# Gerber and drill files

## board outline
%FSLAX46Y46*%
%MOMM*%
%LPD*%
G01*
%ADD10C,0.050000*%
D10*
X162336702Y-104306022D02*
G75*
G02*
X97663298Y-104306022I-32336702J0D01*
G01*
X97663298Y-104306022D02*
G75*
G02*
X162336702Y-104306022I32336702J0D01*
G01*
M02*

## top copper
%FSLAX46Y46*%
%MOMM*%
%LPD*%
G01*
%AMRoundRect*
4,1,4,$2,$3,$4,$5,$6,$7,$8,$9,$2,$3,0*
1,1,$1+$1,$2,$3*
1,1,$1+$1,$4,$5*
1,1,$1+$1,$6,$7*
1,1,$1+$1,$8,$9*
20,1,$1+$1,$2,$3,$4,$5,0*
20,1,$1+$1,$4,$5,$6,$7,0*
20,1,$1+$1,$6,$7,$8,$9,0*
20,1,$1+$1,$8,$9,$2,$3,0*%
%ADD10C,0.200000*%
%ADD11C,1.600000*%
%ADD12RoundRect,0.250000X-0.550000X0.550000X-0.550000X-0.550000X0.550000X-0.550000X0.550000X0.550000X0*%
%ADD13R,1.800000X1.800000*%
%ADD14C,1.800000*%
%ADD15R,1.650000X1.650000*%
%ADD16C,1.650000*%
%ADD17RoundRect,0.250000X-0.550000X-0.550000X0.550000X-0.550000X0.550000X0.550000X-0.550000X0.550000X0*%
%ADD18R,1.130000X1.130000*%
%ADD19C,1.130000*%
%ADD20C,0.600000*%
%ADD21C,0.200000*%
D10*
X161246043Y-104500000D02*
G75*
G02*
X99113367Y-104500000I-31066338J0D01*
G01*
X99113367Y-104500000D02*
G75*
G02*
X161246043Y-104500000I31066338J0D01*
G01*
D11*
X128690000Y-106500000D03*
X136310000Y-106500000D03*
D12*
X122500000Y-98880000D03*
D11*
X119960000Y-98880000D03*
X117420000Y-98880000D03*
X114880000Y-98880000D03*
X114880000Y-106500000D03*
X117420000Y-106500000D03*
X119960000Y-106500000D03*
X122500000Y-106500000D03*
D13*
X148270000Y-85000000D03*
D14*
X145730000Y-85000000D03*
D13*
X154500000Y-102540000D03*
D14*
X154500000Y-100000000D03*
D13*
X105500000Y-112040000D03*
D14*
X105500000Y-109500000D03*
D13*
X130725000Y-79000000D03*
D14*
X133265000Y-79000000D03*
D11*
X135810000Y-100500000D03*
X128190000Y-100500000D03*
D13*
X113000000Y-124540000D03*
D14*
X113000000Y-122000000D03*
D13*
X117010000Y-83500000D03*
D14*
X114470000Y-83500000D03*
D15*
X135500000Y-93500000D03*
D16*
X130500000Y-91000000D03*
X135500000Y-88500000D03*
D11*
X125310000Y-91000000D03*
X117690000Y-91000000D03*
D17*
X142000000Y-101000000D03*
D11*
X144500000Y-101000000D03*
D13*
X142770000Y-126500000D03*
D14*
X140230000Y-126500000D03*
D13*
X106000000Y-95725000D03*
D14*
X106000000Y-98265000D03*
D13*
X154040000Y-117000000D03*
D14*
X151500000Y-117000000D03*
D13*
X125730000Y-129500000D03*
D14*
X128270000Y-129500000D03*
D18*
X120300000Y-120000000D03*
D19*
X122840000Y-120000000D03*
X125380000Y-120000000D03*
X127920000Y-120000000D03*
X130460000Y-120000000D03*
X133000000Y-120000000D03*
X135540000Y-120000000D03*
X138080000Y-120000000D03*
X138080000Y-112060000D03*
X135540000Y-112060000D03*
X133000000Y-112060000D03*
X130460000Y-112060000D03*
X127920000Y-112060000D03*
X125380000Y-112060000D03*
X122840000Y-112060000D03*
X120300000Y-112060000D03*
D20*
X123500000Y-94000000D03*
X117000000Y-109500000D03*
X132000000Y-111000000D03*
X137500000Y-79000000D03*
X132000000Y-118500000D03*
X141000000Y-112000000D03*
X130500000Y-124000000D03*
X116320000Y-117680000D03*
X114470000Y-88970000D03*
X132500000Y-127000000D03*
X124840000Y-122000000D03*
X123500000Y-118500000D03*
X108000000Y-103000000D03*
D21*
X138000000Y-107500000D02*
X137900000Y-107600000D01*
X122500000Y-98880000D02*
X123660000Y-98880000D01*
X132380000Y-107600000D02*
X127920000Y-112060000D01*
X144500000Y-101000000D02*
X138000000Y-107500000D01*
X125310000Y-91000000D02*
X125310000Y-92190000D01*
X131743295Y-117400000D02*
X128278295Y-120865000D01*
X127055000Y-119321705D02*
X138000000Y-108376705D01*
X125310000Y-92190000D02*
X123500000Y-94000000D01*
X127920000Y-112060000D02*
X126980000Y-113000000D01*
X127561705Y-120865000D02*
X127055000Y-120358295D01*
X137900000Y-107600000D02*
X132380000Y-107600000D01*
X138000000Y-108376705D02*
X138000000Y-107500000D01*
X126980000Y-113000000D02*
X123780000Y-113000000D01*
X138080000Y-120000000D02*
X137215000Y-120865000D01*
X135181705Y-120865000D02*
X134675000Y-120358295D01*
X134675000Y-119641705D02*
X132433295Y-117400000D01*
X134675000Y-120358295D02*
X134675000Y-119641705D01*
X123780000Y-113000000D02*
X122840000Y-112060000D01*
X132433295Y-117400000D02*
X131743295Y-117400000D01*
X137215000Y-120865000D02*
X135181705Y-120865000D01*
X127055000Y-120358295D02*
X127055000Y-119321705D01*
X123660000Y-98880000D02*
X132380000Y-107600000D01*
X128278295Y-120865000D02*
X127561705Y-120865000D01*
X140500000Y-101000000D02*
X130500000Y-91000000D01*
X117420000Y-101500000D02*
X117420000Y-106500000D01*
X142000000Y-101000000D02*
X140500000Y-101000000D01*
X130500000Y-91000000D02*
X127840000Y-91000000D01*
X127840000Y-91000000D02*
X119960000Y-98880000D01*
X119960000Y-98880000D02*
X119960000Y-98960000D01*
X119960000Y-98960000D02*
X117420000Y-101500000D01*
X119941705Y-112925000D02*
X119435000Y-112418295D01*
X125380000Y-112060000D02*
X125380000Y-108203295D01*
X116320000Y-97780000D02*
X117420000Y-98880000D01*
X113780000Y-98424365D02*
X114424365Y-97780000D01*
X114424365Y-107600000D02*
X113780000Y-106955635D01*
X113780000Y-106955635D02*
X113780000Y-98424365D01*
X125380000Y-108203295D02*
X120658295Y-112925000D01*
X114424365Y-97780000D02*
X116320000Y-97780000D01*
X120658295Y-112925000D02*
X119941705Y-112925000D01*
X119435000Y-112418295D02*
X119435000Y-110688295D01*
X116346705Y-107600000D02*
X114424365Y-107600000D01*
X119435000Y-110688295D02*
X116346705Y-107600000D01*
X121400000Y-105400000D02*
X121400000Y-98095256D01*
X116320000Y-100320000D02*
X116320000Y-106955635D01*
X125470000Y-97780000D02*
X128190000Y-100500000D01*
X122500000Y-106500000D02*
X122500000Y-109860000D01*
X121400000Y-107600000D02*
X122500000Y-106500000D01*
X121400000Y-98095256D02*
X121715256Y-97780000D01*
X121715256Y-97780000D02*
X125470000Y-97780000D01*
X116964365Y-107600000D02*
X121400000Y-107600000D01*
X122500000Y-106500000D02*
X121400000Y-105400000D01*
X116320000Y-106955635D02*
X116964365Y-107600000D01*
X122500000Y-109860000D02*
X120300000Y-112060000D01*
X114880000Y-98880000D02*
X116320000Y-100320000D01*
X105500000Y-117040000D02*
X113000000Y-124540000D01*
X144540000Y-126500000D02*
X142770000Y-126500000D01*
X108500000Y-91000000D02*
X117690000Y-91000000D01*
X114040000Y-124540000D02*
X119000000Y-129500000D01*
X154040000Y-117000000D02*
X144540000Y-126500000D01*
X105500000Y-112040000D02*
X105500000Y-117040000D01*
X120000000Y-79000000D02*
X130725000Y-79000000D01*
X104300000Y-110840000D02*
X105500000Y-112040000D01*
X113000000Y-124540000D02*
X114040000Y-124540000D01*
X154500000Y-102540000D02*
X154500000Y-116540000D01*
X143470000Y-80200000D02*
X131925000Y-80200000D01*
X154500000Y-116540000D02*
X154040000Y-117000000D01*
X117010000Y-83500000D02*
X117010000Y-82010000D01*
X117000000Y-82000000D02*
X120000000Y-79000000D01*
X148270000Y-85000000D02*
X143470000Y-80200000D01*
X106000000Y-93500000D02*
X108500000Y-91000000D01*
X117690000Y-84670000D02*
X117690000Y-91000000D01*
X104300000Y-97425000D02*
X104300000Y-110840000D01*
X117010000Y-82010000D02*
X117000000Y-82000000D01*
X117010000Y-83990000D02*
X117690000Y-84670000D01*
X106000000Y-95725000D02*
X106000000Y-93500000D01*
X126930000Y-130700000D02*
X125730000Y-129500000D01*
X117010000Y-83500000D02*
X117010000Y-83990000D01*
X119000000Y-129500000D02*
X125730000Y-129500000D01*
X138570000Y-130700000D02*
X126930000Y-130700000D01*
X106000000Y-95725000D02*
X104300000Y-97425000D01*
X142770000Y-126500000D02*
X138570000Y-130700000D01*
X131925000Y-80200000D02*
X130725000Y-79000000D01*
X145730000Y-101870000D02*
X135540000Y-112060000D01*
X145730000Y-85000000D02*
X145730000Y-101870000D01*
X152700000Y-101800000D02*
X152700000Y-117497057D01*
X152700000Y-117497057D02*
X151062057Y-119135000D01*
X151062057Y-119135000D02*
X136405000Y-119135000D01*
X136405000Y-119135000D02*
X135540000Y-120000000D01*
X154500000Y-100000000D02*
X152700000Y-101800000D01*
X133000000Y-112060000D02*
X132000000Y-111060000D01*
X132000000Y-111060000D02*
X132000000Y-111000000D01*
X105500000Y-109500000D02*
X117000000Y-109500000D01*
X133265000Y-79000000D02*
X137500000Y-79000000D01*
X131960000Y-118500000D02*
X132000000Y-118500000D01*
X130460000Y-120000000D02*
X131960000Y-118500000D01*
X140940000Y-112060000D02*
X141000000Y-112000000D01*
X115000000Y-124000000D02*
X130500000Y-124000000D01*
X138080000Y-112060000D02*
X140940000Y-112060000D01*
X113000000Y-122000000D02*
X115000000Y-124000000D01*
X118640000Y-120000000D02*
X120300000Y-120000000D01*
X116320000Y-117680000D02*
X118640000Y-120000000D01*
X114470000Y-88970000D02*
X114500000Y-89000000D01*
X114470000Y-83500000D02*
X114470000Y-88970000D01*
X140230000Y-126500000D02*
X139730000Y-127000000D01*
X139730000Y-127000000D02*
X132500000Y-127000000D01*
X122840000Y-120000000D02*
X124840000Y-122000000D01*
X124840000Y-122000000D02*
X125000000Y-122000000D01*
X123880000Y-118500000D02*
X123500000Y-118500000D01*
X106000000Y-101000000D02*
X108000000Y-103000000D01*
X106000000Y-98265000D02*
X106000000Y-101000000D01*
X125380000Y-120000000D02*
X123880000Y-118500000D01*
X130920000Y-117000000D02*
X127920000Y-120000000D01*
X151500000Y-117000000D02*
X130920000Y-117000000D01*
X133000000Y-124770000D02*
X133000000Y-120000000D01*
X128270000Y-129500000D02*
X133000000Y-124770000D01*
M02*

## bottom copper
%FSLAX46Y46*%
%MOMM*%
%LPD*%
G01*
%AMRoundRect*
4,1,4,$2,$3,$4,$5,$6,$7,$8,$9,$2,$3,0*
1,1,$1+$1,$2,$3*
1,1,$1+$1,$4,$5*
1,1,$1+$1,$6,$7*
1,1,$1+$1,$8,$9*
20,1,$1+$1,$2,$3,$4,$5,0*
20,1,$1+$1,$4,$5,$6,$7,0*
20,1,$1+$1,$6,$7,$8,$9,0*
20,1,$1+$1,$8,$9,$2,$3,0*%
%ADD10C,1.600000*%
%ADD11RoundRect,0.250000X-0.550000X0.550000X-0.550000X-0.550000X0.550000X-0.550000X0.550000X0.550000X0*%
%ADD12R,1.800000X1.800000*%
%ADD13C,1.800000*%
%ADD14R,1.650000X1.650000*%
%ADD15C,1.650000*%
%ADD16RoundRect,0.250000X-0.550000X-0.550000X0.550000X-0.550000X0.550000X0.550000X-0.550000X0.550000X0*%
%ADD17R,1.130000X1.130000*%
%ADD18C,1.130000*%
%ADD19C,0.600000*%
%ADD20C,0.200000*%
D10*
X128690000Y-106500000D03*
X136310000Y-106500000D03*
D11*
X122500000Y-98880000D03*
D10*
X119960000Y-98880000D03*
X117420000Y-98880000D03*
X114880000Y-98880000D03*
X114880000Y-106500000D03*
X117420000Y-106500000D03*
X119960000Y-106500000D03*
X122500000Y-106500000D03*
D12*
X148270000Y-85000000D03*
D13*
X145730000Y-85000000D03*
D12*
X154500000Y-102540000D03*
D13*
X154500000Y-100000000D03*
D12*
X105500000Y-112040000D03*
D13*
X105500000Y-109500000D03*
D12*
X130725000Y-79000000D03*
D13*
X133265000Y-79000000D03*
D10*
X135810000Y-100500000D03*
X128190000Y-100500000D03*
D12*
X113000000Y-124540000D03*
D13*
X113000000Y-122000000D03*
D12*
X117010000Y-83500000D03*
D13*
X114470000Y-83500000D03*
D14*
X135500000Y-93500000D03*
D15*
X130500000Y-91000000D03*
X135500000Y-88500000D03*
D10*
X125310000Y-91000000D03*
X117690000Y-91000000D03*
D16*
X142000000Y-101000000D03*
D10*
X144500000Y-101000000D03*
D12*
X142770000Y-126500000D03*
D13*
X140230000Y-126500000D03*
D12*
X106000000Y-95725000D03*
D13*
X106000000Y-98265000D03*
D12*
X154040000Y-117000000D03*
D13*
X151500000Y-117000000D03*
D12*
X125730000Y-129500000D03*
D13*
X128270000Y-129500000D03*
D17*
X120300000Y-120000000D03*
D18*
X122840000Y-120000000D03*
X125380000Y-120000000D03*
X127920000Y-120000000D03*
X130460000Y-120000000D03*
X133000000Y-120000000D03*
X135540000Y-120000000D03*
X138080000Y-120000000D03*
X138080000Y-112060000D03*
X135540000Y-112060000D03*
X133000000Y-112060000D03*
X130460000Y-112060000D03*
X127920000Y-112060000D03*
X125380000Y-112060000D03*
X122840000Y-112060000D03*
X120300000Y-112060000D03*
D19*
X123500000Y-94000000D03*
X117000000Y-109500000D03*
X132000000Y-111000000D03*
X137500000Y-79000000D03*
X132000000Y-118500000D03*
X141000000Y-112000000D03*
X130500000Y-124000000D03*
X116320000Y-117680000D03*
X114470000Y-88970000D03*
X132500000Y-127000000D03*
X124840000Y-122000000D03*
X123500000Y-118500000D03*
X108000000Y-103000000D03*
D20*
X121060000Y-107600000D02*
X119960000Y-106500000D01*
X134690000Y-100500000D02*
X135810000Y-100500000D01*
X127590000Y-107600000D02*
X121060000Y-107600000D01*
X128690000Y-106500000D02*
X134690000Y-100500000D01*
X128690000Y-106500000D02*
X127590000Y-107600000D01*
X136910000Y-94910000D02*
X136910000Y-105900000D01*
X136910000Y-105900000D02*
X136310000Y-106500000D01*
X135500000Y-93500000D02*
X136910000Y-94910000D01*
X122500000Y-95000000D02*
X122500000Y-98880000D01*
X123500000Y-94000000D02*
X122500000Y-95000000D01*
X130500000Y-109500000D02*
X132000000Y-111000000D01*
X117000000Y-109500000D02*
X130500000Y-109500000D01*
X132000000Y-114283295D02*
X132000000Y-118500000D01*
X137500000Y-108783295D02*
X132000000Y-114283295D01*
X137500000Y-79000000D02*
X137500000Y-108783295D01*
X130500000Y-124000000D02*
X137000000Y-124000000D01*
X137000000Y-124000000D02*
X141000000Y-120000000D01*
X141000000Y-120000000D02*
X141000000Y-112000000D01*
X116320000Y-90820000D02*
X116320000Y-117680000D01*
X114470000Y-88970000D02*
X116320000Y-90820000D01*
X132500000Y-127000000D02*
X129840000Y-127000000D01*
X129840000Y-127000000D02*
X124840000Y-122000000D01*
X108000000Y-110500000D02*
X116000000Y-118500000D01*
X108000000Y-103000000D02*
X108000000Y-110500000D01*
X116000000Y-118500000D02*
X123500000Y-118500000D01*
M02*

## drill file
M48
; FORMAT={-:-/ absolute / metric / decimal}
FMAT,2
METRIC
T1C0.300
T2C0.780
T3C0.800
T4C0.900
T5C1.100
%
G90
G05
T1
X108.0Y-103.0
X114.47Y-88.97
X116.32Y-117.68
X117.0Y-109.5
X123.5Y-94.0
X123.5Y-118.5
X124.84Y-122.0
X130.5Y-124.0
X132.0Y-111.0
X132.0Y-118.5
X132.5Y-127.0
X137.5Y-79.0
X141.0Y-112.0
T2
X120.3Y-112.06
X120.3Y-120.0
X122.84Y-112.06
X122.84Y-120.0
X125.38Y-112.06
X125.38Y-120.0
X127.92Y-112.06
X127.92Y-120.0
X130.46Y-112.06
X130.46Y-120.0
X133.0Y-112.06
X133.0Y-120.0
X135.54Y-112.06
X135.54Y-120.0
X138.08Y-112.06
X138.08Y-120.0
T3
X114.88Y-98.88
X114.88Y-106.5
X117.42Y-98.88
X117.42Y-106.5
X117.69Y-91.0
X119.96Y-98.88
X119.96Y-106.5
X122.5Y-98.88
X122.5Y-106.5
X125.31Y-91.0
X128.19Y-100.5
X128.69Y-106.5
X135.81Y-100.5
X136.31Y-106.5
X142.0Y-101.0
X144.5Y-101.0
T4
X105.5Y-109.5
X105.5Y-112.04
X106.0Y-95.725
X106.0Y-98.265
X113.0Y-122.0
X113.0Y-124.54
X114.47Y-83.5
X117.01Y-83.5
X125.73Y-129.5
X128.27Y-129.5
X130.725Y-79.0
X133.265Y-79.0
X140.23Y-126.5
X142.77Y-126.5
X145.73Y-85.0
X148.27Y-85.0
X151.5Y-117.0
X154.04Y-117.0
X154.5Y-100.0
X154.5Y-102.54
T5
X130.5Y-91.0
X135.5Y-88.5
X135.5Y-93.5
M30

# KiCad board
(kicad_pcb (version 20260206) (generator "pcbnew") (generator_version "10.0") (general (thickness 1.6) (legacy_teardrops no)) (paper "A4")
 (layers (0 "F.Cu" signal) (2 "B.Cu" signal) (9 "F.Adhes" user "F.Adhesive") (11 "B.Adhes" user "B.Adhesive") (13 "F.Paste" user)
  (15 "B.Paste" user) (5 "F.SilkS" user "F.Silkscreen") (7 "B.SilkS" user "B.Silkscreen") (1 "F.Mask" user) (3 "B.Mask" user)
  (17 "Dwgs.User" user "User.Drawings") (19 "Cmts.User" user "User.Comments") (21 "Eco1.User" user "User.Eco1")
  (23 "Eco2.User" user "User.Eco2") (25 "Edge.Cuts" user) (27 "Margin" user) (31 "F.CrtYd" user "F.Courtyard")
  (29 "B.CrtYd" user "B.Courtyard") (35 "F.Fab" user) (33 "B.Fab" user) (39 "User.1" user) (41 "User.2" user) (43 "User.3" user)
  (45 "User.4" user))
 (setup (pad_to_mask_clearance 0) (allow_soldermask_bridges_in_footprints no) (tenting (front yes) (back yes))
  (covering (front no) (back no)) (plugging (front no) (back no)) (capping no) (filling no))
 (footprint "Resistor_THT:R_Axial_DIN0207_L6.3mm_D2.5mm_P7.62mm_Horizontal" (layer "F.Cu") (at 128.69 106.5)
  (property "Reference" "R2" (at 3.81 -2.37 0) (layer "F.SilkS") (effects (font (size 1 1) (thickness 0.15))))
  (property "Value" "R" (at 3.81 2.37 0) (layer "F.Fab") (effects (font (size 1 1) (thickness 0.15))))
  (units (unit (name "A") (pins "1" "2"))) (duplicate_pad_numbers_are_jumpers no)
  (pad "1" thru_hole circle (at 0 0) (size 1.6 1.6) (drill 0.8) (layers "*.Cu" "*.Mask") (remove_unused_layers no) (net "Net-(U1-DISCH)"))
  (pad "2" thru_hole circle (at 7.62 0) (size 1.6 1.6) (drill 0.8) (layers "*.Cu" "*.Mask") (remove_unused_layers no) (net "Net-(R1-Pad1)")))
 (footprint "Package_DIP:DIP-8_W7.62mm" (layer "F.Cu") (at 122.5 98.88 -90)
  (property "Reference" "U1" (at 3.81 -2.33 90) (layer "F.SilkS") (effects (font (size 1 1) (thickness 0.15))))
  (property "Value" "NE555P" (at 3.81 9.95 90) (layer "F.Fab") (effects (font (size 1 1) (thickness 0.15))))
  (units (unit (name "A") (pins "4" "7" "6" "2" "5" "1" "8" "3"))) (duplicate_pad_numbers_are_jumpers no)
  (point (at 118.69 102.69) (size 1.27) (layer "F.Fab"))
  (pad "1" thru_hole roundrect (at 0 0 270) (size 1.6 1.6) (drill 0.8) (layers "*.Cu" "*.Mask") (remove_unused_layers no)
   (roundrect_rratio 0.15625) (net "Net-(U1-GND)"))
  (pad "2" thru_hole circle (at 0 2.54 270) (size 1.6 1.6) (drill 0.8) (layers "*.Cu" "*.Mask") (remove_unused_layers no)
   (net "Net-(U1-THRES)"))
  (pad "3" thru_hole circle (at 0 5.08 270) (size 1.6 1.6) (drill 0.8) (layers "*.Cu" "*.Mask") (remove_unused_layers no)
   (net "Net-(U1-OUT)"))
  (pad "4" thru_hole circle (at 0 7.62 270) (size 1.6 1.6) (drill 0.8) (layers "*.Cu" "*.Mask") (remove_unused_layers no)
   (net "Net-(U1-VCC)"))
  (pad "5" thru_hole circle (at 7.62 7.62 270) (size 1.6 1.6) (drill 0.8) (layers "*.Cu" "*.Mask") (remove_unused_layers no)
   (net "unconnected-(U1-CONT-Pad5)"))
  (pad "6" thru_hole circle (at 7.62 5.08 270) (size 1.6 1.6) (drill 0.8) (layers "*.Cu" "*.Mask") (remove_unused_layers no)
   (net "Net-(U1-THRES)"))
  (pad "7" thru_hole circle (at 7.62 2.54 270) (size 1.6 1.6) (drill 0.8) (layers "*.Cu" "*.Mask") (remove_unused_layers no)
   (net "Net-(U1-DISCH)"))
  (pad "8" thru_hole circle (at 7.62 0 270) (size 1.6 1.6) (drill 0.8) (layers "*.Cu" "*.Mask") (remove_unused_layers no)
   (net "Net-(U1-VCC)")))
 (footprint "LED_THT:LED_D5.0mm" (layer "F.Cu") (at 148.27 85 180)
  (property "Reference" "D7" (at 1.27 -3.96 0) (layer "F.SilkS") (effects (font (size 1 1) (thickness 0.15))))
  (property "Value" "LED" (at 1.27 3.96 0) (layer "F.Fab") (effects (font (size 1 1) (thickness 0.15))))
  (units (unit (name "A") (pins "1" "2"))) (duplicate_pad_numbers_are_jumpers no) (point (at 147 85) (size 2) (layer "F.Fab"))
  (pad "1" thru_hole rect (at 0 0 180) (size 1.8 1.8) (drill 0.9) (layers "*.Cu" "*.Mask") (remove_unused_layers no) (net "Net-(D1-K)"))
  (pad "2" thru_hole circle (at 2.54 0 180) (size 1.8 1.8) (drill 0.9) (layers "*.Cu" "*.Mask") (remove_unused_layers no) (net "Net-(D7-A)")))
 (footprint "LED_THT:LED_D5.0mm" (layer "F.Cu") (at 154.5 102.54 90)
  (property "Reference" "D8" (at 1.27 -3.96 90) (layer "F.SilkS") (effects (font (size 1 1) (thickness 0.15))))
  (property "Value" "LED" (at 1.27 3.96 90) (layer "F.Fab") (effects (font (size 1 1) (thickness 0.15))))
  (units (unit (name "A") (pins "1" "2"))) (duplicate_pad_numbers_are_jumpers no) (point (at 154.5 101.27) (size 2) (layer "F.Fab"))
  (pad "1" thru_hole rect (at 0 0 90) (size 1.8 1.8) (drill 0.9) (layers "*.Cu" "*.Mask") (remove_unused_layers no) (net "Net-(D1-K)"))
  (pad "2" thru_hole circle (at 2.54 0 90) (size 1.8 1.8) (drill 0.9) (layers "*.Cu" "*.Mask") (remove_unused_layers no) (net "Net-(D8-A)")))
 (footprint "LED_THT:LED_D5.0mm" (layer "F.Cu") (at 105.5 112.04 90)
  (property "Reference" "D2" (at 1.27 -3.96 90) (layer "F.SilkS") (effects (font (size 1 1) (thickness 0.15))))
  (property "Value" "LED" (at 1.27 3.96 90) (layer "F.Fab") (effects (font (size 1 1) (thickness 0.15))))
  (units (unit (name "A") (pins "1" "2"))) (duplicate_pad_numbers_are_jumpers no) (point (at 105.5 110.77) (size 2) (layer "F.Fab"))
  (pad "1" thru_hole rect (at 0 0 90) (size 1.8 1.8) (drill 0.9) (layers "*.Cu" "*.Mask") (remove_unused_layers no) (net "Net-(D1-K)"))
  (pad "2" thru_hole circle (at 2.54 0 90) (size 1.8 1.8) (drill 0.9) (layers "*.Cu" "*.Mask") (remove_unused_layers no) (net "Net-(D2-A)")))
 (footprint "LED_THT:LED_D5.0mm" (layer "F.Cu") (at 130.725 79)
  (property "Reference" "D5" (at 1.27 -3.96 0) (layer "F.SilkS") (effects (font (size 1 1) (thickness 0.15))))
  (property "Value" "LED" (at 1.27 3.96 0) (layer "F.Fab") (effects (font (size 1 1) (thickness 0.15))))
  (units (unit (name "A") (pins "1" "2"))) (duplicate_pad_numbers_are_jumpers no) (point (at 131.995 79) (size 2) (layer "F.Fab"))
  (pad "1" thru_hole rect (at 0 0) (size 1.8 1.8) (drill 0.9) (layers "*.Cu" "*.Mask") (remove_unused_layers no) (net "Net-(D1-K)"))
  (pad "2" thru_hole circle (at 2.54 0) (size 1.8 1.8) (drill 0.9) (layers "*.Cu" "*.Mask") (remove_unused_layers no) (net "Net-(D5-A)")))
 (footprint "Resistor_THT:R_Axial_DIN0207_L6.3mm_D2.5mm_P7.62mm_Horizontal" (layer "F.Cu") (at 135.81 100.5 180)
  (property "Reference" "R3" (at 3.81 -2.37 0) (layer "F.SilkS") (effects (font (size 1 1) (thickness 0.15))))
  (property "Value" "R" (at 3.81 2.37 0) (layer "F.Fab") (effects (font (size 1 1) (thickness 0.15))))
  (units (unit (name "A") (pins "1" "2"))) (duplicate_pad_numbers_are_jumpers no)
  (pad "1" thru_hole circle (at 0 0 180) (size 1.6 1.6) (drill 0.8) (layers "*.Cu" "*.Mask") (remove_unused_layers no)
   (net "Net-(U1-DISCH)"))
  (pad "2" thru_hole circle (at 7.62 0 180) (size 1.6 1.6) (drill 0.8) (layers "*.Cu" "*.Mask") (remove_unused_layers no)
   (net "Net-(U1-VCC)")))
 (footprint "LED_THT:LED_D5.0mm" (layer "F.Cu") (at 113 124.54 90)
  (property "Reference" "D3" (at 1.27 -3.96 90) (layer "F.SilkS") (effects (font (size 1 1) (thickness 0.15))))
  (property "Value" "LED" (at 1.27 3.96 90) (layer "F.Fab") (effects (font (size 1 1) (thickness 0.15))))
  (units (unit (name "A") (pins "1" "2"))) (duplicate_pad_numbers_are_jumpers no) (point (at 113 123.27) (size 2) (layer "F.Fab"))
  (pad "1" thru_hole rect (at 0 0 90) (size 1.8 1.8) (drill 0.9) (layers "*.Cu" "*.Mask") (remove_unused_layers no) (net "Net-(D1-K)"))
  (pad "2" thru_hole circle (at 2.54 0 90) (size 1.8 1.8) (drill 0.9) (layers "*.Cu" "*.Mask") (remove_unused_layers no) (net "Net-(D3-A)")))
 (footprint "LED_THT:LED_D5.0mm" (layer "F.Cu") (at 117.01 83.5 180)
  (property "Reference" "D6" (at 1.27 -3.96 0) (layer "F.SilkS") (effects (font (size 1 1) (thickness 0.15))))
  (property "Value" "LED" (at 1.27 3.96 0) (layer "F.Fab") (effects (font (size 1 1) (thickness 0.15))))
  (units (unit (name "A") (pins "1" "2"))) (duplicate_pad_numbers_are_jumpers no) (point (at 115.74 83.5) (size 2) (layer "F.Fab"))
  (pad "1" thru_hole rect (at 0 0 180) (size 1.8 1.8) (drill 0.9) (layers "*.Cu" "*.Mask") (remove_unused_layers no) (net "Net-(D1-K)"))
  (pad "2" thru_hole circle (at 2.54 0 180) (size 1.8 1.8) (drill 0.9) (layers "*.Cu" "*.Mask") (remove_unused_layers no) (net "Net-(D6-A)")))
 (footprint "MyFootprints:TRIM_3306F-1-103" (layer "F.Cu") (at 133 91)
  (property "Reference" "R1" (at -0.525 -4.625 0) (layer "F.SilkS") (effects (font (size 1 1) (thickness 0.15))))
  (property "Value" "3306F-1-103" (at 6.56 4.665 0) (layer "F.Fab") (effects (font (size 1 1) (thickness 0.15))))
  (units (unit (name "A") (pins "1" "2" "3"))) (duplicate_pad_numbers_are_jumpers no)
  (pad "1" thru_hole rect (at 2.5 2.5) (size 1.65 1.65) (drill 1.1) (layers "*.Cu" "*.Mask") (remove_unused_layers no) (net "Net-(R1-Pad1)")
   (solder_mask_margin 0.102))
  (pad "2" thru_hole circle (at -2.5 0) (size 1.65 1.65) (drill 1.1) (layers "*.Cu" "*.Mask") (remove_unused_layers no)
   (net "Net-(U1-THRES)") (solder_mask_margin 0.102))
  (pad "3" thru_hole circle (at 2.5 -2.5) (size 1.65 1.65) (drill 1.1) (layers "*.Cu" "*.Mask") (remove_unused_layers no)
   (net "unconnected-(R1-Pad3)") (solder_mask_margin 0.102)))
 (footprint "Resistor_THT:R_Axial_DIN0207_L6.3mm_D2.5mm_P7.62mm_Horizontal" (layer "F.Cu") (at 125.31 91 180)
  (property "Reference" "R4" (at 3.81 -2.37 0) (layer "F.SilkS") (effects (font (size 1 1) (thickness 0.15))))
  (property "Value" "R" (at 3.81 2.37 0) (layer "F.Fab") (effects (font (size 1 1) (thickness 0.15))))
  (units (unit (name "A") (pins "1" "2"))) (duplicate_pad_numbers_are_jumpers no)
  (pad "1" thru_hole circle (at 0 0 180) (size 1.6 1.6) (drill 0.8) (layers "*.Cu" "*.Mask") (remove_unused_layers no) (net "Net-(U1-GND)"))
  (pad "2" thru_hole circle (at 7.62 0 180) (size 1.6 1.6) (drill 0.8) (layers "*.Cu" "*.Mask") (remove_unused_layers no) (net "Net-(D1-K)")))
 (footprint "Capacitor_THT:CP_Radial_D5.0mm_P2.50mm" (layer "F.Cu") (at 142 101)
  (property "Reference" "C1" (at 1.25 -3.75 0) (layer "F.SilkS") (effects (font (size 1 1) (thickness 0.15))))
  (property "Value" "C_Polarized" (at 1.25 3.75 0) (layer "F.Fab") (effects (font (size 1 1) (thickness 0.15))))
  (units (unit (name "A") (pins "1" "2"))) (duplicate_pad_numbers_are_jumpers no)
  (pad "1" thru_hole roundrect (at 0 0) (size 1.6 1.6) (drill 0.8) (layers "*.Cu" "*.Mask") (remove_unused_layers no)
   (roundrect_rratio 0.15625) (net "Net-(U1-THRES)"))
  (pad "2" thru_hole circle (at 2.5 0) (size 1.6 1.6) (drill 0.8) (layers "*.Cu" "*.Mask") (remove_unused_layers no) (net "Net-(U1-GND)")))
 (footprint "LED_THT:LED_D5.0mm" (layer "F.Cu") (at 142.77 126.5 180)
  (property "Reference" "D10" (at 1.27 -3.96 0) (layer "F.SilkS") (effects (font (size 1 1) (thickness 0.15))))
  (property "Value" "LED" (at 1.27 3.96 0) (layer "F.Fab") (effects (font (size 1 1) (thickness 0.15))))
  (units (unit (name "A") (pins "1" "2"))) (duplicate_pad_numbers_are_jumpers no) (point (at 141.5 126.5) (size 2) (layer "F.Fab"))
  (pad "1" thru_hole rect (at 0 0 180) (size 1.8 1.8) (drill 0.9) (layers "*.Cu" "*.Mask") (remove_unused_layers no) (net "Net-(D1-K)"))
  (pad "2" thru_hole circle (at 2.54 0 180) (size 1.8 1.8) (drill 0.9) (layers "*.Cu" "*.Mask") (remove_unused_layers no)
   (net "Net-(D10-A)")))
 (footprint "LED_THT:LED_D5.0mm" (layer "F.Cu") (at 106 95.725 -90)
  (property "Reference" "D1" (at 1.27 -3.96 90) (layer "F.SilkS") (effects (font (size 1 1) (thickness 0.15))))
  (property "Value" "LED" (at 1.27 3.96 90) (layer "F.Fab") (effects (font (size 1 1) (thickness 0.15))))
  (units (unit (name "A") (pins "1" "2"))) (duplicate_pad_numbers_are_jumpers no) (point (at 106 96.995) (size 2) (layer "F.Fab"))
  (pad "1" thru_hole rect (at 0 0 270) (size 1.8 1.8) (drill 0.9) (layers "*.Cu" "*.Mask") (remove_unused_layers no) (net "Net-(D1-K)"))
  (pad "2" thru_hole circle (at 2.54 0 270) (size 1.8 1.8) (drill 0.9) (layers "*.Cu" "*.Mask") (remove_unused_layers no) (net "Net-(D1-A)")))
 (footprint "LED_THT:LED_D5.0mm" (layer "F.Cu") (at 154.04 117 180)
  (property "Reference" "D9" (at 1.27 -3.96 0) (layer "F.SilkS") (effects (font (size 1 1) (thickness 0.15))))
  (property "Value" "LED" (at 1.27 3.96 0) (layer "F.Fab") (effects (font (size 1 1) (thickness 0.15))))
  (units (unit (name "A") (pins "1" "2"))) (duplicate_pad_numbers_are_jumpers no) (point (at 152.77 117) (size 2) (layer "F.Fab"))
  (pad "1" thru_hole rect (at 0 0 180) (size 1.8 1.8) (drill 0.9) (layers "*.Cu" "*.Mask") (remove_unused_layers no) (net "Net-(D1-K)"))
  (pad "2" thru_hole circle (at 2.54 0 180) (size 1.8 1.8) (drill 0.9) (layers "*.Cu" "*.Mask") (remove_unused_layers no) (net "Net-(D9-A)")))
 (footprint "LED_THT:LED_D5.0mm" (layer "F.Cu") (at 125.73 129.5)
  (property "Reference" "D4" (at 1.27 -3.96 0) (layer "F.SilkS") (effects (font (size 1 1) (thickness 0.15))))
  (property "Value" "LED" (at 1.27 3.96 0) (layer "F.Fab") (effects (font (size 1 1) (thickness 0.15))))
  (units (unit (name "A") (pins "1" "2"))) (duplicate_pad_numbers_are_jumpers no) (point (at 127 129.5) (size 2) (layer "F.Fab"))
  (pad "1" thru_hole rect (at 0 0) (size 1.8 1.8) (drill 0.9) (layers "*.Cu" "*.Mask") (remove_unused_layers no) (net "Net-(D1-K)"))
  (pad "2" thru_hole circle (at 2.54 0) (size 1.8 1.8) (drill 0.9) (layers "*.Cu" "*.Mask") (remove_unused_layers no) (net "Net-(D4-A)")))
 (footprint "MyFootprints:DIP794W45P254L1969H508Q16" (layer "F.Cu") (at 129.19 116.03 90)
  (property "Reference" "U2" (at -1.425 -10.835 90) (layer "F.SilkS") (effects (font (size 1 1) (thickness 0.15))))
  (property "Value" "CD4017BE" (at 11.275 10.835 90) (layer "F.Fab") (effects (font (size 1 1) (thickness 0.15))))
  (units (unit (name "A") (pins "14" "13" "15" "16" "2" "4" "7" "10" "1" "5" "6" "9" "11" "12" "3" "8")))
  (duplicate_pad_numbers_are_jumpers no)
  (pad "1" thru_hole rect (at -3.97 -8.89 90) (size 1.13 1.13) (drill 0.78) (layers "*.Cu" "*.Mask") (remove_unused_layers no)
   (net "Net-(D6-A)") (solder_mask_margin 0.102))
  (pad "2" thru_hole circle (at -3.97 -6.35 90) (size 1.13 1.13) (drill 0.78) (layers "*.Cu" "*.Mask") (remove_unused_layers no)
   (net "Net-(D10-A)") (solder_mask_margin 0.102))
  (pad "3" thru_hole circle (at -3.97 -3.81 90) (size 1.13 1.13) (drill 0.78) (layers "*.Cu" "*.Mask") (remove_unused_layers no)
   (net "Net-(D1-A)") (solder_mask_margin 0.102))
  (pad "4" thru_hole circle (at -3.97 -1.27 90) (size 1.13 1.13) (drill 0.78) (layers "*.Cu" "*.Mask") (remove_unused_layers no)
   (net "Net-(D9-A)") (solder_mask_margin 0.102))
  (pad "5" thru_hole circle (at -3.97 1.27 90) (size 1.13 1.13) (drill 0.78) (layers "*.Cu" "*.Mask") (remove_unused_layers no)
   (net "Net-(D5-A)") (solder_mask_margin 0.102))
  (pad "6" thru_hole circle (at -3.97 3.81 90) (size 1.13 1.13) (drill 0.78) (layers "*.Cu" "*.Mask") (remove_unused_layers no)
   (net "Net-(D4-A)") (solder_mask_margin 0.102))
  (pad "7" thru_hole circle (at -3.97 6.35 90) (size 1.13 1.13) (drill 0.78) (layers "*.Cu" "*.Mask") (remove_unused_layers no)
   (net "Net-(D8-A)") (solder_mask_margin 0.102))
  (pad "8" thru_hole circle (at -3.97 8.89 90) (size 1.13 1.13) (drill 0.78) (layers "*.Cu" "*.Mask") (remove_unused_layers no)
   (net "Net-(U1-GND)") (solder_mask_margin 0.102))
  (pad "9" thru_hole circle (at 3.97 8.89 90) (size 1.13 1.13) (drill 0.78) (layers "*.Cu" "*.Mask") (remove_unused_layers no)
   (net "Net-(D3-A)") (solder_mask_margin 0.102))
  (pad "10" thru_hole circle (at 3.97 6.35 90) (size 1.13 1.13) (drill 0.78) (layers "*.Cu" "*.Mask") (remove_unused_layers no)
   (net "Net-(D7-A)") (solder_mask_margin 0.102))
  (pad "11" thru_hole circle (at 3.97 3.81 90) (size 1.13 1.13) (drill 0.78) (layers "*.Cu" "*.Mask") (remove_unused_layers no)
   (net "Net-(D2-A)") (solder_mask_margin 0.102))
  (pad "12" thru_hole circle (at 3.97 1.27 90) (size 1.13 1.13) (drill 0.78) (layers "*.Cu" "*.Mask") (remove_unused_layers no)
   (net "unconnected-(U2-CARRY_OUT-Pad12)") (solder_mask_margin 0.102))
  (pad "13" thru_hole circle (at 3.97 -1.27 90) (size 1.13 1.13) (drill 0.78) (layers "*.Cu" "*.Mask") (remove_unused_layers no)
   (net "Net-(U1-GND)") (solder_mask_margin 0.102))
  (pad "14" thru_hole circle (at 3.97 -3.81 90) (size 1.13 1.13) (drill 0.78) (layers "*.Cu" "*.Mask") (remove_unused_layers no)
   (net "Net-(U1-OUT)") (solder_mask_margin 0.102))
  (pad "15" thru_hole circle (at 3.97 -6.35 90) (size 1.13 1.13) (drill 0.78) (layers "*.Cu" "*.Mask") (remove_unused_layers no)
   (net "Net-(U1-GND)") (solder_mask_margin 0.102))
  (pad "16" thru_hole circle (at 3.97 -8.89 90) (size 1.13 1.13) (drill 0.78) (layers "*.Cu" "*.Mask") (remove_unused_layers no)
   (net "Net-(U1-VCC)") (solder_mask_margin 0.102)))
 (gr_circle (center 130.179705 104.5) (end 155.5 122.5) (stroke (width 0.2) (type default)) (fill no) (layer "F.Cu"))
 (gr_circle (center 130 104.306022) (end 101 90) (stroke (width 0.05) (type default)) (fill no) (layer "Edge.Cuts"))
 (segment (start 121.06 107.6) (end 119.96 106.5) (width 0.2) (layer "B.Cu") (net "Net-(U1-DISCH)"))
 (segment (start 134.69 100.5) (end 135.81 100.5) (width 0.2) (layer "B.Cu") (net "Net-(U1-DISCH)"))
 (segment (start 127.59 107.6) (end 121.06 107.6) (width 0.2) (layer "B.Cu") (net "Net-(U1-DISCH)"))
 (segment (start 128.69 106.5) (end 134.69 100.5) (width 0.2) (layer "B.Cu") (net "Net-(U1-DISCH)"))
 (segment (start 128.69 106.5) (end 127.59 107.6) (width 0.2) (layer "B.Cu") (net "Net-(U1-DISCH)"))
 (segment (start 136.91 94.91) (end 136.91 105.9) (width 0.2) (layer "B.Cu") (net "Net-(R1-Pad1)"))
 (segment (start 136.91 105.9) (end 136.31 106.5) (width 0.2) (layer "B.Cu") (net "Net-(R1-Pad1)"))
 (segment (start 135.5 93.5) (end 136.91 94.91) (width 0.2) (layer "B.Cu") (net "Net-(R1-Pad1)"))
 (segment (start 138 107.5) (end 137.9 107.6) (width 0.2) (layer "F.Cu") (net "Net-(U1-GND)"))
 (segment (start 122.5 98.88) (end 123.66 98.88) (width 0.2) (layer "F.Cu") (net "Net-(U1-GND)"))
 (segment (start 132.38 107.6) (end 127.92 112.06) (width 0.2) (layer "F.Cu") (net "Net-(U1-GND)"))
 (segment (start 144.5 101) (end 138 107.5) (width 0.2) (layer "F.Cu") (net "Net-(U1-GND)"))
 (segment (start 125.31 91) (end 125.31 92.19) (width 0.2) (layer "F.Cu") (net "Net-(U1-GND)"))
 (segment (start 131.743295 117.4) (end 128.278295 120.865) (width 0.2) (layer "F.Cu") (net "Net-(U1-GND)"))
 (segment (start 127.055 119.321705) (end 138 108.376705) (width 0.2) (layer "F.Cu") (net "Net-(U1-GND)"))
 (segment (start 125.31 92.19) (end 123.5 94) (width 0.2) (layer "F.Cu") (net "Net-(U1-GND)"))
 (segment (start 127.92 112.06) (end 126.98 113) (width 0.2) (layer "F.Cu") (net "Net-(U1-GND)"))
 (segment (start 127.561705 120.865) (end 127.055 120.358295) (width 0.2) (layer "F.Cu") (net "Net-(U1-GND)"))
 (segment (start 137.9 107.6) (end 132.38 107.6) (width 0.2) (layer "F.Cu") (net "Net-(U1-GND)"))
 (segment (start 138 108.376705) (end 138 107.5) (width 0.2) (layer "F.Cu") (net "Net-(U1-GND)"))
 (segment (start 126.98 113) (end 123.78 113) (width 0.2) (layer "F.Cu") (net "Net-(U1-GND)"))
 (segment (start 138.08 120) (end 137.215 120.865) (width 0.2) (layer "F.Cu") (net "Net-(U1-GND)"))
 (segment (start 135.181705 120.865) (end 134.675 120.358295) (width 0.2) (layer "F.Cu") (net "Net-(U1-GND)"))
 (segment (start 134.675 119.641705) (end 132.433295 117.4) (width 0.2) (layer "F.Cu") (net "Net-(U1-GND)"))
 (segment (start 134.675 120.358295) (end 134.675 119.641705) (width 0.2) (layer "F.Cu") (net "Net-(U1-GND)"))
 (segment (start 123.78 113) (end 122.84 112.06) (width 0.2) (layer "F.Cu") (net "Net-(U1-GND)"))
 (segment (start 132.433295 117.4) (end 131.743295 117.4) (width 0.2) (layer "F.Cu") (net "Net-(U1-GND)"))
 (segment (start 137.215 120.865) (end 135.181705 120.865) (width 0.2) (layer "F.Cu") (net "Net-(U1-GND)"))
 (segment (start 127.055 120.358295) (end 127.055 119.321705) (width 0.2) (layer "F.Cu") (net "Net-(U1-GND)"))
 (segment (start 123.66 98.88) (end 132.38 107.6) (width 0.2) (layer "F.Cu") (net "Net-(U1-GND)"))
 (segment (start 128.278295 120.865) (end 127.561705 120.865) (width 0.2) (layer "F.Cu") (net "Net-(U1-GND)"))
 (via (at 123.5 94) (size 0.6) (drill 0.3) (layers "F.Cu" "B.Cu") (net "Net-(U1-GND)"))
 (segment (start 122.5 95) (end 122.5 98.88) (width 0.2) (layer "B.Cu") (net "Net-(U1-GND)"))
 (segment (start 123.5 94) (end 122.5 95) (width 0.2) (layer "B.Cu") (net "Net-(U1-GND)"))
 (segment (start 140.5 101) (end 130.5 91) (width 0.2) (layer "F.Cu") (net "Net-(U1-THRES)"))
 (segment (start 117.42 101.5) (end 117.42 106.5) (width 0.2) (layer "F.Cu") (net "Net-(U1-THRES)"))
 (segment (start 142 101) (end 140.5 101) (width 0.2) (layer "F.Cu") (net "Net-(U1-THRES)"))
 (segment (start 130.5 91) (end 127.84 91) (width 0.2) (layer "F.Cu") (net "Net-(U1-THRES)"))
 (segment (start 127.84 91) (end 119.96 98.88) (width 0.2) (layer "F.Cu") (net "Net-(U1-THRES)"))
 (segment (start 119.96 98.88) (end 119.96 98.96) (width 0.2) (layer "F.Cu") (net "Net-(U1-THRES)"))
 (segment (start 119.96 98.96) (end 117.42 101.5) (width 0.2) (layer "F.Cu") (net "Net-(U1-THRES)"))
 (segment (start 119.941705 112.925) (end 119.435 112.418295) (width 0.2) (layer "F.Cu") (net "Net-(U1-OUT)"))
 (segment (start 125.38 112.06) (end 125.38 108.203295) (width 0.2) (layer "F.Cu") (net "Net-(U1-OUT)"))
 (segment (start 116.32 97.78) (end 117.42 98.88) (width 0.2) (layer "F.Cu") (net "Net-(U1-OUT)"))
 (segment (start 113.78 98.424365) (end 114.424365 97.78) (width 0.2) (layer "F.Cu") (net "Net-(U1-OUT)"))
 (segment (start 114.424365 107.6) (end 113.78 106.955635) (width 0.2) (layer "F.Cu") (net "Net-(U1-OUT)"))
 (segment (start 113.78 106.955635) (end 113.78 98.424365) (width 0.2) (layer "F.Cu") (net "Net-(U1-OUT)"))
 (segment (start 125.38 108.203295) (end 120.658295 112.925) (width 0.2) (layer "F.Cu") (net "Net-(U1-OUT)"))
 (segment (start 114.424365 97.78) (end 116.32 97.78) (width 0.2) (layer "F.Cu") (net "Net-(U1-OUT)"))
 (segment (start 120.658295 112.925) (end 119.941705 112.925) (width 0.2) (layer "F.Cu") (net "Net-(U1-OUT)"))
 (segment (start 119.435 112.418295) (end 119.435 110.688295) (width 0.2) (layer "F.Cu") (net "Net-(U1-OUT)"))
 (segment (start 116.346705 107.6) (end 114.424365 107.6) (width 0.2) (layer "F.Cu") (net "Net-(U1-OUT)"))
 (segment (start 119.435 110.688295) (end 116.346705 107.6) (width 0.2) (layer "F.Cu") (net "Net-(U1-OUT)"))
 (segment (start 121.4 105.4) (end 121.4 98.095256) (width 0.2) (layer "F.Cu") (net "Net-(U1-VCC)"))
 (segment (start 116.32 100.32) (end 116.32 106.955635) (width 0.2) (layer "F.Cu") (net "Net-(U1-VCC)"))
 (segment (start 125.47 97.78) (end 128.19 100.5) (width 0.2) (layer "F.Cu") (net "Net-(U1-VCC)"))
 (segment (start 122.5 106.5) (end 122.5 109.86) (width 0.2) (layer "F.Cu") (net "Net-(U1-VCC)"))
 (segment (start 121.4 107.6) (end 122.5 106.5) (width 0.2) (layer "F.Cu") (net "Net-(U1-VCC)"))
 (segment (start 121.4 98.095256) (end 121.715256 97.78) (width 0.2) (layer "F.Cu") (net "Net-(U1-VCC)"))
 (segment (start 121.715256 97.78) (end 125.47 97.78) (width 0.2) (layer "F.Cu") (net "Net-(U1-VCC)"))
 (segment (start 116.964365 107.6) (end 121.4 107.6) (width 0.2) (layer "F.Cu") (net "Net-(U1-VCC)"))
 (segment (start 122.5 106.5) (end 121.4 105.4) (width 0.2) (layer "F.Cu") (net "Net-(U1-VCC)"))
 (segment (start 116.32 106.955635) (end 116.964365 107.6) (width 0.2) (layer "F.Cu") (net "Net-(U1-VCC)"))
 (segment (start 122.5 109.86) (end 120.3 112.06) (width 0.2) (layer "F.Cu") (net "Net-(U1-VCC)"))
 (segment (start 114.88 98.88) (end 116.32 100.32) (width 0.2) (layer "F.Cu") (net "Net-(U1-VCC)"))
 (segment (start 105.5 117.04) (end 113 124.54) (width 0.2) (layer "F.Cu") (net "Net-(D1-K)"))
 (segment (start 144.54 126.5) (end 142.77 126.5) (width 0.2) (layer "F.Cu") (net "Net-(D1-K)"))
 (segment (start 108.5 91) (end 117.69 91) (width 0.2) (layer "F.Cu") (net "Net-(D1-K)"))
 (segment (start 114.04 124.54) (end 119 129.5) (width 0.2) (layer "F.Cu") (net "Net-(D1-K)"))
 (segment (start 154.04 117) (end 144.54 126.5) (width 0.2) (layer "F.Cu") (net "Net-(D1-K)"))
 (segment (start 105.5 112.04) (end 105.5 117.04) (width 0.2) (layer "F.Cu") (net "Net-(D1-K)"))
 (segment (start 120 79) (end 130.725 79) (width 0.2) (layer "F.Cu") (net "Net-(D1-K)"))
 (segment (start 104.3 110.84) (end 105.5 112.04) (width 0.2) (layer "F.Cu") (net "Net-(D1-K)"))
 (segment (start 113 124.54) (end 114.04 124.54) (width 0.2) (layer "F.Cu") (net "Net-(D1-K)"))
 (segment (start 154.5 102.54) (end 154.5 116.54) (width 0.2) (layer "F.Cu") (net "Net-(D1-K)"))
 (segment (start 143.47 80.2) (end 131.925 80.2) (width 0.2) (layer "F.Cu") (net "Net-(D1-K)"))
 (segment (start 154.5 116.54) (end 154.04 117) (width 0.2) (layer "F.Cu") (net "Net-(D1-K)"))
 (segment (start 117.01 83.5) (end 117.01 82.01) (width 0.2) (layer "F.Cu") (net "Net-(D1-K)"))
 (segment (start 117 82) (end 120 79) (width 0.2) (layer "F.Cu") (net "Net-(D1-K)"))
 (segment (start 148.27 85) (end 143.47 80.2) (width 0.2) (layer "F.Cu") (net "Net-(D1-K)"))
 (segment (start 106 93.5) (end 108.5 91) (width 0.2) (layer "F.Cu") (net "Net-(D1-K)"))
 (segment (start 117.69 84.67) (end 117.69 91) (width 0.2) (layer "F.Cu") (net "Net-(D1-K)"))
 (segment (start 104.3 97.425) (end 104.3 110.84) (width 0.2) (layer "F.Cu") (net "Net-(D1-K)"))
 (segment (start 117.01 82.01) (end 117 82) (width 0.2) (layer "F.Cu") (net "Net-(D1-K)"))
 (segment (start 117.01 83.99) (end 117.69 84.67) (width 0.2) (layer "F.Cu") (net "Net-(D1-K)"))
 (segment (start 106 95.725) (end 106 93.5) (width 0.2) (layer "F.Cu") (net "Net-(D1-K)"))
 (segment (start 126.93 130.7) (end 125.73 129.5) (width 0.2) (layer "F.Cu") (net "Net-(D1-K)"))
 (segment (start 117.01 83.5) (end 117.01 83.99) (width 0.2) (layer "F.Cu") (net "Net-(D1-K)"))
 (segment (start 119 129.5) (end 125.73 129.5) (width 0.2) (layer "F.Cu") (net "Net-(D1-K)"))
 (segment (start 138.57 130.7) (end 126.93 130.7) (width 0.2) (layer "F.Cu") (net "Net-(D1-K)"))
 (segment (start 106 95.725) (end 104.3 97.425) (width 0.2) (layer "F.Cu") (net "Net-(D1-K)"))
 (segment (start 142.77 126.5) (end 138.57 130.7) (width 0.2) (layer "F.Cu") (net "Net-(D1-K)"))
 (segment (start 131.925 80.2) (end 130.725 79) (width 0.2) (layer "F.Cu") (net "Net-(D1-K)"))
 (segment (start 145.73 101.87) (end 135.54 112.06) (width 0.2) (layer "F.Cu") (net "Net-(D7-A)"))
 (segment (start 145.73 85) (end 145.73 101.87) (width 0.2) (layer "F.Cu") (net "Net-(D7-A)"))
 (segment (start 152.7 101.8) (end 152.7 117.497057) (width 0.2) (layer "F.Cu") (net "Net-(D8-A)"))
 (segment (start 152.7 117.497057) (end 151.062057 119.135) (width 0.2) (layer "F.Cu") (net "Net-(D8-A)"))
 (segment (start 151.062057 119.135) (end 136.405 119.135) (width 0.2) (layer "F.Cu") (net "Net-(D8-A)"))
 (segment (start 136.405 119.135) (end 135.54 120) (width 0.2) (layer "F.Cu") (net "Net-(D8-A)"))
 (segment (start 154.5 100) (end 152.7 101.8) (width 0.2) (layer "F.Cu") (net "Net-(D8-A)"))
 (segment (start 133 112.06) (end 132 111.06) (width 0.2) (layer "F.Cu") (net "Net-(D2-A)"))
 (segment (start 132 111.06) (end 132 111) (width 0.2) (layer "F.Cu") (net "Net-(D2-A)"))
 (segment (start 105.5 109.5) (end 117 109.5) (width 0.2) (layer "F.Cu") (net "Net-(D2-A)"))
 (via (at 117 109.5) (size 0.6) (drill 0.3) (layers "F.Cu" "B.Cu") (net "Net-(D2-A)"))
 (via (at 132 111) (size 0.6) (drill 0.3) (layers "F.Cu" "B.Cu") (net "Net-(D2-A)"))
 (segment (start 130.5 109.5) (end 132 111) (width 0.2) (layer "B.Cu") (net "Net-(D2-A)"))
 (segment (start 117 109.5) (end 130.5 109.5) (width 0.2) (layer "B.Cu") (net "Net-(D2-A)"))
 (segment (start 133.265 79) (end 137.5 79) (width 0.2) (layer "F.Cu") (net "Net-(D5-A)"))
 (segment (start 131.96 118.5) (end 132 118.5) (width 0.2) (layer "F.Cu") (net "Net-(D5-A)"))
 (segment (start 130.46 120) (end 131.96 118.5) (width 0.2) (layer "F.Cu") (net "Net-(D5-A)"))
 (via (at 137.5 79) (size 0.6) (drill 0.3) (layers "F.Cu" "B.Cu") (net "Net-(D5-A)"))
 (via (at 132 118.5) (size 0.6) (drill 0.3) (layers "F.Cu" "B.Cu") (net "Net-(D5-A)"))
 (segment (start 132 114.283295) (end 132 118.5) (width 0.2) (layer "B.Cu") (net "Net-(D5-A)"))
 (segment (start 137.5 108.783295) (end 132 114.283295) (width 0.2) (layer "B.Cu") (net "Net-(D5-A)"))
 (segment (start 137.5 79) (end 137.5 108.783295) (width 0.2) (layer "B.Cu") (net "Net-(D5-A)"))
 (segment (start 140.94 112.06) (end 141 112) (width 0.2) (layer "F.Cu") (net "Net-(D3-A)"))
 (segment (start 115 124) (end 130.5 124) (width 0.2) (layer "F.Cu") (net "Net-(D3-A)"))
 (segment (start 138.08 112.06) (end 140.94 112.06) (width 0.2) (layer "F.Cu") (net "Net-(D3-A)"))
 (segment (start 113 122) (end 115 124) (width 0.2) (layer "F.Cu") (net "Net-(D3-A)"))
 (via (at 141 112) (size 0.6) (drill 0.3) (layers "F.Cu" "B.Cu") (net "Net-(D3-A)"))
 (via (at 130.5 124) (size 0.6) (drill 0.3) (layers "F.Cu" "B.Cu") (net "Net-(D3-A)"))
 (segment (start 130.5 124) (end 137 124) (width 0.2) (layer "B.Cu") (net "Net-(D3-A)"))
 (segment (start 137 124) (end 141 120) (width 0.2) (layer "B.Cu") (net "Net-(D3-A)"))
 (segment (start 141 120) (end 141 112) (width 0.2) (layer "B.Cu") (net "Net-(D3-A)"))
 (segment (start 118.64 120) (end 120.3 120) (width 0.2) (layer "F.Cu") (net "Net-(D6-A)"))
 (segment (start 116.32 117.68) (end 118.64 120) (width 0.2) (layer "F.Cu") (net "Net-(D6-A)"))
 (segment (start 114.47 88.97) (end 114.5 89) (width 0.2) (layer "F.Cu") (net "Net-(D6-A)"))
 (segment (start 114.47 83.5) (end 114.47 88.97) (width 0.2) (layer "F.Cu") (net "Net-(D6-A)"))
 (via (at 116.32 117.68) (size 0.6) (drill 0.3) (layers "F.Cu" "B.Cu") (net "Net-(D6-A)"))
 (via (at 114.47 88.97) (size 0.6) (drill 0.3) (layers "F.Cu" "B.Cu") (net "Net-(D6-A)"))
 (segment (start 116.32 90.82) (end 116.32 117.68) (width 0.2) (layer "B.Cu") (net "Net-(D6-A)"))
 (segment (start 114.47 88.97) (end 116.32 90.82) (width 0.2) (layer "B.Cu") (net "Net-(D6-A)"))
 (segment (start 140.23 126.5) (end 139.73 127) (width 0.2) (layer "F.Cu") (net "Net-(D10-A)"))
 (segment (start 139.73 127) (end 132.5 127) (width 0.2) (layer "F.Cu") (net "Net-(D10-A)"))
 (segment (start 122.84 120) (end 124.84 122) (width 0.2) (layer "F.Cu") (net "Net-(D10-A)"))
 (segment (start 124.84 122) (end 125 122) (width 0.2) (layer "F.Cu") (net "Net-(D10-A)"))
 (via (at 132.5 127) (size 0.6) (drill 0.3) (layers "F.Cu" "B.Cu") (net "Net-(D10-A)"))
 (via (at 124.84 122) (size 0.6) (drill 0.3) (layers "F.Cu" "B.Cu") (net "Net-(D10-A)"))
 (segment (start 132.5 127) (end 129.84 127) (width 0.2) (layer "B.Cu") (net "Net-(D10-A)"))
 (segment (start 129.84 127) (end 124.84 122) (width 0.2) (layer "B.Cu") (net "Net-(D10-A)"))
 (segment (start 123.88 118.5) (end 123.5 118.5) (width 0.2) (layer "F.Cu") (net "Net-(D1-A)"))
 (segment (start 106 101) (end 108 103) (width 0.2) (layer "F.Cu") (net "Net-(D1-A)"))
 (segment (start 106 98.265) (end 106 101) (width 0.2) (layer "F.Cu") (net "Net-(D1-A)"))
 (segment (start 125.38 120) (end 123.88 118.5) (width 0.2) (layer "F.Cu") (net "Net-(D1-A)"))
 (via (at 123.5 118.5) (size 0.6) (drill 0.3) (layers "F.Cu" "B.Cu") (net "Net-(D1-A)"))
 (via (at 108 103) (size 0.6) (drill 0.3) (layers "F.Cu" "B.Cu") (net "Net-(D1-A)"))
 (segment (start 108 110.5) (end 116 118.5) (width 0.2) (layer "B.Cu") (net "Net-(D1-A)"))
 (segment (start 108 103) (end 108 110.5) (width 0.2) (layer "B.Cu") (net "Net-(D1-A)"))
 (segment (start 116 118.5) (end 123.5 118.5) (width 0.2) (layer "B.Cu") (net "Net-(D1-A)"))
 (segment (start 130.92 117) (end 127.92 120) (width 0.2) (layer "F.Cu") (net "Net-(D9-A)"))
 (segment (start 151.5 117) (end 130.92 117) (width 0.2) (layer "F.Cu") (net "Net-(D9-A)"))
 (segment (start 133 124.77) (end 133 120) (width 0.2) (layer "F.Cu") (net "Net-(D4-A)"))
 (segment (start 128.27 129.5) (end 133 124.77) (width 0.2) (layer "F.Cu") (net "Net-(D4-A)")))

